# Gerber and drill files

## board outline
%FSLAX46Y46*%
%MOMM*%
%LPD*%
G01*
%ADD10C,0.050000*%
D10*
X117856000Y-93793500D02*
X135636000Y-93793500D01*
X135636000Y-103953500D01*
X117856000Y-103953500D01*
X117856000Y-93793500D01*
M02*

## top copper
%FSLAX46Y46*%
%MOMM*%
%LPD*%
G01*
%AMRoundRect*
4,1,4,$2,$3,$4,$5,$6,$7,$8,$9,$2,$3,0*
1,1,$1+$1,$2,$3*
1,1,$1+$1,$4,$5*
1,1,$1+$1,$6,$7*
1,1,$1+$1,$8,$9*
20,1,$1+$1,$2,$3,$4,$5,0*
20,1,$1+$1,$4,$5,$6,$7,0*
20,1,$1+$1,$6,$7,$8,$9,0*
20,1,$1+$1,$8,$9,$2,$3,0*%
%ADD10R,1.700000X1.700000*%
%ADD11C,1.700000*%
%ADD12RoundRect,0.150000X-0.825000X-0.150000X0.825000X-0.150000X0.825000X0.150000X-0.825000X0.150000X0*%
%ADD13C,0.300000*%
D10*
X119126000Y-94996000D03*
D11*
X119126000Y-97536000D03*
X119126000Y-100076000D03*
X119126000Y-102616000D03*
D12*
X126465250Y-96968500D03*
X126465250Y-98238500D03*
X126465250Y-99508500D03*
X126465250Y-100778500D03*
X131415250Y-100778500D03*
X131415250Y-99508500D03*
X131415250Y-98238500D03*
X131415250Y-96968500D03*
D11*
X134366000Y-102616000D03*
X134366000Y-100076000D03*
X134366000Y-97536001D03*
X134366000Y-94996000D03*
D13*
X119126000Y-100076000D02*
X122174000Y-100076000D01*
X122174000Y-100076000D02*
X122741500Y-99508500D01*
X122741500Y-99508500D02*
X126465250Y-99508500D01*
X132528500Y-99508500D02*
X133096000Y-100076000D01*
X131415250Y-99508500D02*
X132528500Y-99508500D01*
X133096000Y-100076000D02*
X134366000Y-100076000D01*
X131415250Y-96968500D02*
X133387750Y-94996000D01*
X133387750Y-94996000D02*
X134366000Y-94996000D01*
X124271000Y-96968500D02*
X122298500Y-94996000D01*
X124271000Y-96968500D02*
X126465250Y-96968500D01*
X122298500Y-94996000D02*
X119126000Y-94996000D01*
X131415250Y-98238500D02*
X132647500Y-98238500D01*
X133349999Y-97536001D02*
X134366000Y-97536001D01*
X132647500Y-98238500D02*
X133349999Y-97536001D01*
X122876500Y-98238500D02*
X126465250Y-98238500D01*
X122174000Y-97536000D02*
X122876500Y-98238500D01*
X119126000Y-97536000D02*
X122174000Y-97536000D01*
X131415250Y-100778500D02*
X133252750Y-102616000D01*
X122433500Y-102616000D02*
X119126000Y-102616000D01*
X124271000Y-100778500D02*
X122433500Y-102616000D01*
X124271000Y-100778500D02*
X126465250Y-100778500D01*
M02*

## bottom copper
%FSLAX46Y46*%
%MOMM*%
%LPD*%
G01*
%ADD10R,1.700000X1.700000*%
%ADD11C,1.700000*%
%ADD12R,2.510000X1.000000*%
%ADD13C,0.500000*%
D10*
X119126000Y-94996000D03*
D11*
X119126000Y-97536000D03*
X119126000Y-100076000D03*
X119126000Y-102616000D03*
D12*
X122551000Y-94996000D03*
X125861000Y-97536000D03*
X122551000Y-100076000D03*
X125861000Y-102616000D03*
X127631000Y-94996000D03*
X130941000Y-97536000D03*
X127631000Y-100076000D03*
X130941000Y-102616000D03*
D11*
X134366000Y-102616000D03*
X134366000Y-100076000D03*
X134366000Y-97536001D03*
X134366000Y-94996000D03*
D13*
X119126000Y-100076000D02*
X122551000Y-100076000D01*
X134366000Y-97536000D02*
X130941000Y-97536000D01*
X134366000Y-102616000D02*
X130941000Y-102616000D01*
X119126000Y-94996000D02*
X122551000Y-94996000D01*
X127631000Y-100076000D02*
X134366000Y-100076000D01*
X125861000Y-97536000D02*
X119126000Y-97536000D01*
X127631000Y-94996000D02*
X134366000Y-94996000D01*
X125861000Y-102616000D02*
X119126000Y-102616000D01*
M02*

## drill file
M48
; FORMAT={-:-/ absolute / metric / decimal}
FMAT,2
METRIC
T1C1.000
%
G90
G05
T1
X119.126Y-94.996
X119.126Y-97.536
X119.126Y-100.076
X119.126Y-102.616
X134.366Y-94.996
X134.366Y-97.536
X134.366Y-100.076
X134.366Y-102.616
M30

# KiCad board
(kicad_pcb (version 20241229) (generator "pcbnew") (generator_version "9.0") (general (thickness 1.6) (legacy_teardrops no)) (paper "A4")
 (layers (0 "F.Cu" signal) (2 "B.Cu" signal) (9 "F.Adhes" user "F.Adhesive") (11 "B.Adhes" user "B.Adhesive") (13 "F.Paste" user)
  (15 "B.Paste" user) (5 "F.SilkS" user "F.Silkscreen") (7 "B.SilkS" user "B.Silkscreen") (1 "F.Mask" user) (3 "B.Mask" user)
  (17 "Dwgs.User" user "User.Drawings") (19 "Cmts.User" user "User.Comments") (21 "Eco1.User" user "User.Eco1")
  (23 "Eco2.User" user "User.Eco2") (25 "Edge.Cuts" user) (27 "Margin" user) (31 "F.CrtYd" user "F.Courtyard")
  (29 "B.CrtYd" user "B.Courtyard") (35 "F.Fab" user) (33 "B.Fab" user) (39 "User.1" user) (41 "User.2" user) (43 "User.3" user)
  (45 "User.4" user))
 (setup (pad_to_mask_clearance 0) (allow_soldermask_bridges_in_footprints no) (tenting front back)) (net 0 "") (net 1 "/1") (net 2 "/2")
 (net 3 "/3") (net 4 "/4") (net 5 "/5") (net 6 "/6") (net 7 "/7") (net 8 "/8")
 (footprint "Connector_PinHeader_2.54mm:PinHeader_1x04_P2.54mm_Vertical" (layer "F.Cu") (at 119.126 94.996)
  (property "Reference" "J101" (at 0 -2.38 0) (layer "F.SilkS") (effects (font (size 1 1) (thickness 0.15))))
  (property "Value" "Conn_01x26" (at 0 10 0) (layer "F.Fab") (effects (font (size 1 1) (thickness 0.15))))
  (pad "1" thru_hole rect (at 0 0) (size 1.7 1.7) (drill 1) (layers "*.Cu" "*.Mask") (remove_unused_layers no) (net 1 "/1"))
  (pad "2" thru_hole circle (at 0 2.54) (size 1.7 1.7) (drill 1) (layers "*.Cu" "*.Mask") (remove_unused_layers no) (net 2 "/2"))
  (pad "3" thru_hole circle (at 0 5.08) (size 1.7 1.7) (drill 1) (layers "*.Cu" "*.Mask") (remove_unused_layers no) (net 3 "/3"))
  (pad "4" thru_hole circle (at 0 7.62) (size 1.7 1.7) (drill 1) (layers "*.Cu" "*.Mask") (remove_unused_layers no) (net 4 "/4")))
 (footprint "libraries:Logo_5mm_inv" (layer "F.Cu") (at 128.94025 98.8735 90)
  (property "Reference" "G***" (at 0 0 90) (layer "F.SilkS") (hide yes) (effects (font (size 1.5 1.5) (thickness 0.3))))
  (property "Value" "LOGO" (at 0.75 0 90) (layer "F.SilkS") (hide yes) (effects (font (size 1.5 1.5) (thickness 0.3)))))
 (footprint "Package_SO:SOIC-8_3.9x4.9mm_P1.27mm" (layer "F.Cu") (at 128.94025 98.8735)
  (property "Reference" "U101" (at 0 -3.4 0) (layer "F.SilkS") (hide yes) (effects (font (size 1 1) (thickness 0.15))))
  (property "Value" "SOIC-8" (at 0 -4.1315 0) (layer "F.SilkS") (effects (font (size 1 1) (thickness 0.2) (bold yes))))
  (pad "1" smd roundrect (at -2.475 -1.905) (size 1.95 0.6) (layers "F.Cu" "F.Mask" "F.Paste") (roundrect_rratio 0.25) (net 1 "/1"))
  (pad "2" smd roundrect (at -2.475 -0.635) (size 1.95 0.6) (layers "F.Cu" "F.Mask" "F.Paste") (roundrect_rratio 0.25) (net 2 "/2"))
  (pad "3" smd roundrect (at -2.475 0.635) (size 1.95 0.6) (layers "F.Cu" "F.Mask" "F.Paste") (roundrect_rratio 0.25) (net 3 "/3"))
  (pad "4" smd roundrect (at -2.475 1.905) (size 1.95 0.6) (layers "F.Cu" "F.Mask" "F.Paste") (roundrect_rratio 0.25) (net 4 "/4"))
  (pad "5" smd roundrect (at 2.475 1.905) (size 1.95 0.6) (layers "F.Cu" "F.Mask" "F.Paste") (roundrect_rratio 0.25) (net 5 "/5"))
  (pad "6" smd roundrect (at 2.475 0.635) (size 1.95 0.6) (layers "F.Cu" "F.Mask" "F.Paste") (roundrect_rratio 0.25) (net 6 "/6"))
  (pad "7" smd roundrect (at 2.475 -0.635) (size 1.95 0.6) (layers "F.Cu" "F.Mask" "F.Paste") (roundrect_rratio 0.25) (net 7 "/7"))
  (pad "8" smd roundrect (at 2.475 -1.905) (size 1.95 0.6) (layers "F.Cu" "F.Mask" "F.Paste") (roundrect_rratio 0.25) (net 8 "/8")))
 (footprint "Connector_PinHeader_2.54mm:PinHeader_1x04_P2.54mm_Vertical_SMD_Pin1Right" (layer "B.Cu") (at 124.206 98.806 180)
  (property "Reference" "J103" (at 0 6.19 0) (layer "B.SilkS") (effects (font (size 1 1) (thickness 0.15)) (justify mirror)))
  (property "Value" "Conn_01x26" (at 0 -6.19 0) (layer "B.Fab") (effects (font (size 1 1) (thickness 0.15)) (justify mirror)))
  (pad "1" smd rect (at 1.655 3.81 180) (size 2.51 1) (layers "B.Cu" "B.Mask" "B.Paste") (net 1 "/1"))
  (pad "2" smd rect (at -1.655 1.27 180) (size 2.51 1) (layers "B.Cu" "B.Mask" "B.Paste") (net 2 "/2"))
  (pad "3" smd rect (at 1.655 -1.27 180) (size 2.51 1) (layers "B.Cu" "B.Mask" "B.Paste") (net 3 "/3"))
  (pad "4" smd rect (at -1.655 -3.81 180) (size 2.51 1) (layers "B.Cu" "B.Mask" "B.Paste") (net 4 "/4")))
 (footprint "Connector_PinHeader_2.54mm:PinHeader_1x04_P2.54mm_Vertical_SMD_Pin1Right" (layer "B.Cu") (at 129.286 98.806 180)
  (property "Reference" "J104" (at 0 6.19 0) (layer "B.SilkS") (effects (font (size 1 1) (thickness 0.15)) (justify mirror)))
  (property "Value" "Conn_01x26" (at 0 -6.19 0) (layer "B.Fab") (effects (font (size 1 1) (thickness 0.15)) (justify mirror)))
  (pad "1" smd rect (at 1.655 3.81 180) (size 2.51 1) (layers "B.Cu" "B.Mask" "B.Paste") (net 5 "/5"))
  (pad "2" smd rect (at -1.655 1.27 180) (size 2.51 1) (layers "B.Cu" "B.Mask" "B.Paste") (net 6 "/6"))
  (pad "3" smd rect (at 1.655 -1.27 180) (size 2.51 1) (layers "B.Cu" "B.Mask" "B.Paste") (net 7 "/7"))
  (pad "4" smd rect (at -1.655 -3.81 180) (size 2.51 1) (layers "B.Cu" "B.Mask" "B.Paste") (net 8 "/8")))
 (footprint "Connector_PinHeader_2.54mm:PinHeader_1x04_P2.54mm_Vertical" (layer "B.Cu") (at 134.366 102.616)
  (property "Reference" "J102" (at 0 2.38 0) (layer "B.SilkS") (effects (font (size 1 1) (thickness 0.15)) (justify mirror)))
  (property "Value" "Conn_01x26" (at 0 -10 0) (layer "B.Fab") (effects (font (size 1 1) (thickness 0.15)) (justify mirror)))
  (pad "1" thru_hole circle (at 0 0) (size 1.7 1.7) (drill 1) (layers "*.Cu" "*.Mask") (remove_unused_layers no) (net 5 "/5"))
  (pad "2" thru_hole circle (at 0 -2.54) (size 1.7 1.7) (drill 1) (layers "*.Cu" "*.Mask") (remove_unused_layers no) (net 6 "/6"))
  (pad "3" thru_hole circle (at 0 -5.079999) (size 1.7 1.7) (drill 1) (layers "*.Cu" "*.Mask") (remove_unused_layers no) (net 7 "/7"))
  (pad "4" thru_hole circle (at 0 -7.62) (size 1.7 1.7) (drill 1) (layers "*.Cu" "*.Mask") (remove_unused_layers no) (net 8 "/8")))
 (gr_rect (start 117.856 93.7935) (end 135.636 103.9535) (stroke (width 0.05) (type default)) (fill no) (layer "Edge.Cuts"))
 (segment (start 119.126 100.076) (end 122.174 100.076) (width 0.3) (layer "F.Cu") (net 3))
 (segment (start 122.174 100.076) (end 122.7415 99.5085) (width 0.3) (layer "F.Cu") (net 3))
 (segment (start 122.7415 99.5085) (end 126.46525 99.5085) (width 0.3) (layer "F.Cu") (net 3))
 (segment (start 119.126 100.076) (end 122.551 100.076) (width 0.5) (layer "B.Cu") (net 3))
 (segment (start 132.5285 99.5085) (end 133.096 100.076) (width 0.3) (layer "F.Cu") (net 6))
 (segment (start 131.41525 99.5085) (end 132.5285 99.5085) (width 0.3) (layer "F.Cu") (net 6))
 (segment (start 133.096 100.076) (end 134.366 100.076) (width 0.3) (layer "F.Cu") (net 6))
 (segment (start 134.366 97.536) (end 130.941 97.536) (width 0.5) (layer "B.Cu") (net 6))
 (segment (start 131.41525 96.9685) (end 133.38775 94.996) (width 0.3) (layer "F.Cu") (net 8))
 (segment (start 133.38775 94.996) (end 134.366 94.996) (width 0.3) (layer "F.Cu") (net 8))
 (segment (start 134.366 102.616) (end 130.941 102.616) (width 0.5) (layer "B.Cu") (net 8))
 (segment (start 124.271 96.9685) (end 122.2985 94.996) (width 0.3) (layer "F.Cu") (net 1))
 (segment (start 124.271 96.9685) (end 126.46525 96.9685) (width 0.3) (layer "F.Cu") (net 1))
 (segment (start 122.2985 94.996) (end 119.126 94.996) (width 0.3) (layer "F.Cu") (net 1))
 (segment (start 119.126 94.996) (end 122.551 94.996) (width 0.5) (layer "B.Cu") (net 1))
 (segment (start 131.41525 98.2385) (end 132.6475 98.2385) (width 0.3) (layer "F.Cu") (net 7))
 (segment (start 133.349999 97.536001) (end 134.366 97.536001) (width 0.3) (layer "F.Cu") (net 7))
 (segment (start 132.6475 98.2385) (end 133.349999 97.536001) (width 0.3) (layer "F.Cu") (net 7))
 (segment (start 127.631 100.076) (end 134.366 100.076) (width 0.5) (layer "B.Cu") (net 7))
 (segment (start 122.8765 98.2385) (end 126.46525 98.2385) (width 0.3) (layer "F.Cu") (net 2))
 (segment (start 122.174 97.536) (end 122.8765 98.2385) (width 0.3) (layer "F.Cu") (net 2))
 (segment (start 119.126 97.536) (end 122.174 97.536) (width 0.3) (layer "F.Cu") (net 2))
 (segment (start 125.861 97.536) (end 119.126 97.536) (width 0.5) (layer "B.Cu") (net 2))
 (segment (start 131.41525 100.7785) (end 133.25275 102.616) (width 0.3) (layer "F.Cu") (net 5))
 (segment (start 127.631 94.996) (end 134.366 94.996) (width 0.5) (layer "B.Cu") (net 5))
 (segment (start 122.4335 102.616) (end 119.126 102.616) (width 0.3) (layer "F.Cu") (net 4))
 (segment (start 124.271 100.7785) (end 122.4335 102.616) (width 0.3) (layer "F.Cu") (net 4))
 (segment (start 124.271 100.7785) (end 126.46525 100.7785) (width 0.3) (layer "F.Cu") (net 4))
 (segment (start 125.861 102.616) (end 119.126 102.616) (width 0.5) (layer "B.Cu") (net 4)))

